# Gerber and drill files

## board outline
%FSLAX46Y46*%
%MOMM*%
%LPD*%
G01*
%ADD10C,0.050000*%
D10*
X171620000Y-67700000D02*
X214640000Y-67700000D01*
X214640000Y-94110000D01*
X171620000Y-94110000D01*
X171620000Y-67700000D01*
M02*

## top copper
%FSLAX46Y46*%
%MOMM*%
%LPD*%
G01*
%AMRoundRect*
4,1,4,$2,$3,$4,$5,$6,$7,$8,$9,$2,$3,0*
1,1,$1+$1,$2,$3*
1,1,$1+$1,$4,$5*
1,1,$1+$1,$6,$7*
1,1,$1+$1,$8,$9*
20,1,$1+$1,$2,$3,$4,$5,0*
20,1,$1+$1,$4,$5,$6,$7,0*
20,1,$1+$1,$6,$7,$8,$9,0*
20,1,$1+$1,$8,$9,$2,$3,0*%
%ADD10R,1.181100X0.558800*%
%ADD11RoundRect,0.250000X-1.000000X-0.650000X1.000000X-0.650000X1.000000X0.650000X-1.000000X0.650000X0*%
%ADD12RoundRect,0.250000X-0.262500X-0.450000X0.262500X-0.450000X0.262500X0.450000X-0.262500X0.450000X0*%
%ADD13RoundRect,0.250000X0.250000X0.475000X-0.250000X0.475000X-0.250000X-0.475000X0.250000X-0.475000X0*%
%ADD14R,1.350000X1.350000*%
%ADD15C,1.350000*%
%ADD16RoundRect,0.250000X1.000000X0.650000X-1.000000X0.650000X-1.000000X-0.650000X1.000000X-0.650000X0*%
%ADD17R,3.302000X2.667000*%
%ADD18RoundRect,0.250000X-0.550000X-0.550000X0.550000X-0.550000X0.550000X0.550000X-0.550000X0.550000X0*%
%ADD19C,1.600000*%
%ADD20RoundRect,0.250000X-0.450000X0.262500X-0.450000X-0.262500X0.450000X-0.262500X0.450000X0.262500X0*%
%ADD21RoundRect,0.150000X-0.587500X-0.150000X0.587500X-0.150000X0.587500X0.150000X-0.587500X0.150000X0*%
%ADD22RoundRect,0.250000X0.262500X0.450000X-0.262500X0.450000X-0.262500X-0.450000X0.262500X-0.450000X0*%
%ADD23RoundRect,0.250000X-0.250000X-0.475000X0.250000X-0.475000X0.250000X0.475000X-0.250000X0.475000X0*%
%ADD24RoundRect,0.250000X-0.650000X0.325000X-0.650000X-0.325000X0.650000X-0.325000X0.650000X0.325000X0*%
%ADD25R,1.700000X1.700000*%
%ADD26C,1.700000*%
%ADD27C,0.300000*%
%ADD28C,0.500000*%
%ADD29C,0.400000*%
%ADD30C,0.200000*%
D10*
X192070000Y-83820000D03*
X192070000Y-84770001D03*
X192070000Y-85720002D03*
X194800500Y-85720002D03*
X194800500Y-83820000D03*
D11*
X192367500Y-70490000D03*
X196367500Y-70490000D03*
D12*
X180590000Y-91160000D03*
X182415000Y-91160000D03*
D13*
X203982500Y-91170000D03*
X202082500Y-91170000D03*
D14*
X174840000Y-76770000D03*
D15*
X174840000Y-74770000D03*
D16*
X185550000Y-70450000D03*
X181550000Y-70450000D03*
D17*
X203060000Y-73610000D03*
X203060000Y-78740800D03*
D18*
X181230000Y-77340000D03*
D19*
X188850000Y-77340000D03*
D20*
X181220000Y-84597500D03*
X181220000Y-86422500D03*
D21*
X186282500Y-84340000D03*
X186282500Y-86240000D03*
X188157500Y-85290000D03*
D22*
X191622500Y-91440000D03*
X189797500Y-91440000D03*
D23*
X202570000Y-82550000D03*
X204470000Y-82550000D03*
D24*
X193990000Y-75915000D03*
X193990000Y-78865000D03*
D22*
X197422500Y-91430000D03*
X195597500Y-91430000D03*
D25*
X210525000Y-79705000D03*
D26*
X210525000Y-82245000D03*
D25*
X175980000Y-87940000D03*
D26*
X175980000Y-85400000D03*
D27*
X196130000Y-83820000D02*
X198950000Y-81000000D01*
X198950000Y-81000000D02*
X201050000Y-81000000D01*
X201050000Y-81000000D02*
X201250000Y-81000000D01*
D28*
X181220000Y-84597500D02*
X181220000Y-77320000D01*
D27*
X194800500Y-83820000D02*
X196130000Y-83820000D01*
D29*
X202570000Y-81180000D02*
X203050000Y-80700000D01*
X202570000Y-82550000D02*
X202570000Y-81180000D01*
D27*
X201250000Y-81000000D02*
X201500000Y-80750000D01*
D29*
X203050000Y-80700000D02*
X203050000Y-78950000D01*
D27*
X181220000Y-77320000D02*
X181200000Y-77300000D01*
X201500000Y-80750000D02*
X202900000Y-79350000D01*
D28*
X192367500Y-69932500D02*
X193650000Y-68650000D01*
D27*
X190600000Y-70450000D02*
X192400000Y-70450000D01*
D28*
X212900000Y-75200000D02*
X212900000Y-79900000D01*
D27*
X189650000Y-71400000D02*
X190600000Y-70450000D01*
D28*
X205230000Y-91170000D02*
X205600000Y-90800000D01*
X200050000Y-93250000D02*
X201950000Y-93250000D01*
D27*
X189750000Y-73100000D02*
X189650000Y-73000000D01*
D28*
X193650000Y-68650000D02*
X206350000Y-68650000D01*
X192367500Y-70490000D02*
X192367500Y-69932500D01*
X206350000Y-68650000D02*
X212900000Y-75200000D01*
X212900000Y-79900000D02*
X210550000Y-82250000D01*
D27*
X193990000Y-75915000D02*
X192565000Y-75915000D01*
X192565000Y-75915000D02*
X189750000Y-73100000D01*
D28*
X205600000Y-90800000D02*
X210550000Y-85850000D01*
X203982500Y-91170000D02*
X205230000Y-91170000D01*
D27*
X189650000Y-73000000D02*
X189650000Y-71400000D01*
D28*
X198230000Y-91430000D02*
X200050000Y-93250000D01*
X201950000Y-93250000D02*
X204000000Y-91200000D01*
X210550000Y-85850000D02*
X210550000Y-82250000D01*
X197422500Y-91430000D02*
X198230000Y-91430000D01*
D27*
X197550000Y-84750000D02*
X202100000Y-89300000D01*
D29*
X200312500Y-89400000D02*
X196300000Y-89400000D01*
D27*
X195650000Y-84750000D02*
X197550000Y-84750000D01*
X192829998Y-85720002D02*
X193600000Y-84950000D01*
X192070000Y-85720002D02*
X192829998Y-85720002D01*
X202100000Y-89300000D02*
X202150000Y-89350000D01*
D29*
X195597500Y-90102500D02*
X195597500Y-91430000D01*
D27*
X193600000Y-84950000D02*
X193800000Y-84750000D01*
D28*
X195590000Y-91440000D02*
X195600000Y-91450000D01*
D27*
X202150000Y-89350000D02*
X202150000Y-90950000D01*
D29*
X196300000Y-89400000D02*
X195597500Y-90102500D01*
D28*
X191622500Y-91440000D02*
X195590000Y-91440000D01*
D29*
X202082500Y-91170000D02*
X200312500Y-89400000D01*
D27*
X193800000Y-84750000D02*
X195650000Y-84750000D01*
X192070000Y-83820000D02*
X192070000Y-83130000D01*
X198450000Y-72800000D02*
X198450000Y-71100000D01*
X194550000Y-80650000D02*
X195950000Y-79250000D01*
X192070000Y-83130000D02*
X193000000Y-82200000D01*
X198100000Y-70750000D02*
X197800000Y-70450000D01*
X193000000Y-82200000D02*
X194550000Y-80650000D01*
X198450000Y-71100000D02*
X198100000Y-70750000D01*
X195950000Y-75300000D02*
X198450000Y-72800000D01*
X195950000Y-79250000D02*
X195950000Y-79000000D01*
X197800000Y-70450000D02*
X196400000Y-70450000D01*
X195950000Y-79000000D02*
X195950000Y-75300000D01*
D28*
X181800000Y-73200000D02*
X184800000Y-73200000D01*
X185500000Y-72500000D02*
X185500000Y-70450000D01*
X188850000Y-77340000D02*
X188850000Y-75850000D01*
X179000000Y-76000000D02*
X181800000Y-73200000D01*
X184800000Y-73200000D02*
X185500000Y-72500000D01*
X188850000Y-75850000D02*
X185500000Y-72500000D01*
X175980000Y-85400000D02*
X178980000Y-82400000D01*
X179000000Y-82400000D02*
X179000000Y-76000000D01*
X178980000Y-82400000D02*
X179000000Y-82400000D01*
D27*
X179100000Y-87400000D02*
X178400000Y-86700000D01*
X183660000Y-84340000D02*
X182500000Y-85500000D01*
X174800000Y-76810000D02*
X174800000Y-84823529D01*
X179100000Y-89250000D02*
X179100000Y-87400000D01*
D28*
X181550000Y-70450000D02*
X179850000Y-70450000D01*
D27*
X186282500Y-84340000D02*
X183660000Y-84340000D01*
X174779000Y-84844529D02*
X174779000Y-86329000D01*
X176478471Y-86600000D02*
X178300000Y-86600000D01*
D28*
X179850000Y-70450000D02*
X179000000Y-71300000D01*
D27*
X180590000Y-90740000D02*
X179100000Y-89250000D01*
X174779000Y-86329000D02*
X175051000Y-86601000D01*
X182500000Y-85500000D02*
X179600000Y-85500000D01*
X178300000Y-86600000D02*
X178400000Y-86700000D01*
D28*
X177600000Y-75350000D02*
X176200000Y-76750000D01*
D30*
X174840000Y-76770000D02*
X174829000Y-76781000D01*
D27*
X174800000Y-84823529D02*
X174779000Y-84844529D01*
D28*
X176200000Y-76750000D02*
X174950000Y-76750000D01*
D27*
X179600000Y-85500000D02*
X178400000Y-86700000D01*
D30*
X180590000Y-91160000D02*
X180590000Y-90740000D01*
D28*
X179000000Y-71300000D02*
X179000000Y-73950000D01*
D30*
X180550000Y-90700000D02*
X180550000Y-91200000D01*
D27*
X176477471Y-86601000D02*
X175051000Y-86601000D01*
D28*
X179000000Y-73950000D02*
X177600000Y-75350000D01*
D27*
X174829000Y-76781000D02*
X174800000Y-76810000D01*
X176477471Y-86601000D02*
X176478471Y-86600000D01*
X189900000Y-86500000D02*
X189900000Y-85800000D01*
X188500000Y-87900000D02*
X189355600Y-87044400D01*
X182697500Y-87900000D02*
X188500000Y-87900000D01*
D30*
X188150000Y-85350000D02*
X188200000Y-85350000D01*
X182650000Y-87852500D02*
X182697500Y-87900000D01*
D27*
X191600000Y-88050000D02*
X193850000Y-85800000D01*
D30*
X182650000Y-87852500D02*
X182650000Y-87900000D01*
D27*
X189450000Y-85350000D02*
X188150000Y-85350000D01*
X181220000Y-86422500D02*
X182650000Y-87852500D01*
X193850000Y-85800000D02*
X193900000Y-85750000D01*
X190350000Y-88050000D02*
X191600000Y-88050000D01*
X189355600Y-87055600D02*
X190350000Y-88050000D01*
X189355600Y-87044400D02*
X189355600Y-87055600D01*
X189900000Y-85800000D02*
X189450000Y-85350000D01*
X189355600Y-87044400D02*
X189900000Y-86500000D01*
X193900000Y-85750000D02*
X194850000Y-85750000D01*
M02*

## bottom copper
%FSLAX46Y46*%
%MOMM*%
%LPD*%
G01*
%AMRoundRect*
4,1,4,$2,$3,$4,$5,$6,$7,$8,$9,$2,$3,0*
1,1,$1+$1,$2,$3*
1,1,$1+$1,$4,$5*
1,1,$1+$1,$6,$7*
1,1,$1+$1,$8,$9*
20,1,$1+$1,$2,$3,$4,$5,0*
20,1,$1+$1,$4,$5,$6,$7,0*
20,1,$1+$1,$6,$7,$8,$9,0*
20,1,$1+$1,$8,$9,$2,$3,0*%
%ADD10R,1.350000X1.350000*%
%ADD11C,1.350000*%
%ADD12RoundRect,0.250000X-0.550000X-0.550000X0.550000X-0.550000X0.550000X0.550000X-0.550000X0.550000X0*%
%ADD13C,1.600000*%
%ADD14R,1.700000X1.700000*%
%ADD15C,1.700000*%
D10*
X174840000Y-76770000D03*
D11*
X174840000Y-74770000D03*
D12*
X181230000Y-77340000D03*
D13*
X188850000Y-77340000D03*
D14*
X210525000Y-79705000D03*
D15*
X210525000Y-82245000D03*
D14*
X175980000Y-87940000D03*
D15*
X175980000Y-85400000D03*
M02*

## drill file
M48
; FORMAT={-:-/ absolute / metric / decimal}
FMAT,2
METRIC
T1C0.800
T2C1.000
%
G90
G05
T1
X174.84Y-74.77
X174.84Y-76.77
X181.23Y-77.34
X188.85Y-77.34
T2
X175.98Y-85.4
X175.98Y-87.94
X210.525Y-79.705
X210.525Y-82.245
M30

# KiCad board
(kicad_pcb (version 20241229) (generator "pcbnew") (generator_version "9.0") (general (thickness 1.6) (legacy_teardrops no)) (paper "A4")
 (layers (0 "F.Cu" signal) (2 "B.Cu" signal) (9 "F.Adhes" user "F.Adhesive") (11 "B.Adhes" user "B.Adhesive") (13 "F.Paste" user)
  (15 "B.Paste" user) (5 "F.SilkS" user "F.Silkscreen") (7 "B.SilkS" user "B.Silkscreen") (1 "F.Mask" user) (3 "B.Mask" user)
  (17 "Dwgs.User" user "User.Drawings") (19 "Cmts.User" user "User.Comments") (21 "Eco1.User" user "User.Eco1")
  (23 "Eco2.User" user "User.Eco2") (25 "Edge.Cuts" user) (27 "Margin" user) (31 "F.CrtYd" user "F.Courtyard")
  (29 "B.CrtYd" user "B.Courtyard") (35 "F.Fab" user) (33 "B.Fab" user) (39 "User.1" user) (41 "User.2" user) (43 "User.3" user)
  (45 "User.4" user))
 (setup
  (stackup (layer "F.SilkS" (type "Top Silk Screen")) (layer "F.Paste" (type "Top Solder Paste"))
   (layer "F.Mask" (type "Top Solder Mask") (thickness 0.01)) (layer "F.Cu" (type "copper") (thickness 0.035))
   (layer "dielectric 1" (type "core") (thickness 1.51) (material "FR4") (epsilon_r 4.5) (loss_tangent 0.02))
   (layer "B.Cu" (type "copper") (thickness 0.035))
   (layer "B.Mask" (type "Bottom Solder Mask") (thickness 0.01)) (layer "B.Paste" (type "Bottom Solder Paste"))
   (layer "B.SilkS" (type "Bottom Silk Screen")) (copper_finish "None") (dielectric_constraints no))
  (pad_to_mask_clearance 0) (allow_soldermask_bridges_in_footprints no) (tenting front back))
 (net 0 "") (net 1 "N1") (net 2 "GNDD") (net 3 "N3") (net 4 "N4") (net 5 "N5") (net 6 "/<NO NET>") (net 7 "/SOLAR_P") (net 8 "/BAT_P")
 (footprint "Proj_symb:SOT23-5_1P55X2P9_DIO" (layer "F.Cu") (at 193.43525 84.770001)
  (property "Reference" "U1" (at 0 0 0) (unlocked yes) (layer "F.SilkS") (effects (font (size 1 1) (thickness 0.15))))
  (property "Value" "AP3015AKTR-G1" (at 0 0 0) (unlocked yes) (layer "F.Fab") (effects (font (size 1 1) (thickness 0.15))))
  (pad "1" smd rect (at -1.36525 -0.950001) (size 1.1811 0.5588) (layers "F.Cu" "F.Mask" "F.Paste") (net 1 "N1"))
  (pad "2" smd rect (at -1.36525 0) (size 1.1811 0.5588) (layers "F.Cu" "F.Mask" "F.Paste") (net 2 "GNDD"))
  (pad "3" smd rect (at -1.36525 0.950001) (size 1.1811 0.5588) (layers "F.Cu" "F.Mask" "F.Paste") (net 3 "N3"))
  (pad "4" smd rect (at 1.36525 0.950001) (size 1.1811 0.5588) (layers "F.Cu" "F.Mask" "F.Paste") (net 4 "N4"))
  (pad "5" smd rect (at 1.36525 -0.950001) (size 1.1811 0.5588) (layers "F.Cu" "F.Mask" "F.Paste") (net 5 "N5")))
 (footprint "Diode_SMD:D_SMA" (layer "F.Cu") (at 194.3675 70.49)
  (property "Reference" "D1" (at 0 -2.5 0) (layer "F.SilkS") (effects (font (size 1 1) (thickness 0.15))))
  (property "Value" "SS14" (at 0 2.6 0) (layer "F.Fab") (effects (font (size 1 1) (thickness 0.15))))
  (pad "1" smd roundrect (at -2 0) (size 2.5 1.8) (layers "F.Cu" "F.Mask" "F.Paste") (roundrect_rratio 0.1388888889) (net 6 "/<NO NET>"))
  (pad "2" smd roundrect (at 2 0) (size 2.5 1.8) (layers "F.Cu" "F.Mask" "F.Paste") (roundrect_rratio 0.1388888889) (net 1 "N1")))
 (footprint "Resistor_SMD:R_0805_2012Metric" (layer "F.Cu") (at 181.5025 91.16)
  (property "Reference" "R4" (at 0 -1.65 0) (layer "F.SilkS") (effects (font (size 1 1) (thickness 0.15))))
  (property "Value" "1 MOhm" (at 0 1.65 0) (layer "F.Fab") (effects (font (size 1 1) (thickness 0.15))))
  (pad "1" smd roundrect (at -0.9125 0) (size 1.025 1.4) (layers "F.Cu" "F.Mask" "F.Paste") (roundrect_rratio 0.243902) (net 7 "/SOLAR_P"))
  (pad "2" smd roundrect (at 0.9125 0) (size 1.025 1.4) (layers "F.Cu" "F.Mask" "F.Paste") (roundrect_rratio 0.243902) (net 2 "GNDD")))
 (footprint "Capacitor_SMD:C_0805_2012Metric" (layer "F.Cu") (at 203.0325 91.17 180)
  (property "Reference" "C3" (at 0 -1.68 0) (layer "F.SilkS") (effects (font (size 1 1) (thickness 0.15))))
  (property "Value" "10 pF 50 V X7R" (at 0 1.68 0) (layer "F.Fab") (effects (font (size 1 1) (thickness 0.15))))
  (pad "1" smd roundrect (at -0.95 0 180) (size 1 1.45) (layers "F.Cu" "F.Mask" "F.Paste") (roundrect_rratio 0.25) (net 6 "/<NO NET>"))
  (pad "2" smd roundrect (at 0.95 0 180) (size 1 1.45) (layers "F.Cu" "F.Mask" "F.Paste") (roundrect_rratio 0.25) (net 3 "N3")))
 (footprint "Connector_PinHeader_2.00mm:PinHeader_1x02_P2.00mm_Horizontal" (layer "F.Cu") (at 174.84 76.77 180)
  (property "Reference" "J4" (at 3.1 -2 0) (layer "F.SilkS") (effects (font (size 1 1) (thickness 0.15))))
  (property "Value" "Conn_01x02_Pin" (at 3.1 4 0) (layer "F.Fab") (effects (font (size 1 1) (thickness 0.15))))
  (pad "1" thru_hole rect (at 0 0 180) (size 1.35 1.35) (drill 0.8) (layers "*.Cu" "*.Mask") (remove_unused_layers no) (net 7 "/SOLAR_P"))
  (pad "2" thru_hole circle (at 0 2 180) (size 1.35 1.35) (drill 0.8) (layers "*.Cu" "*.Mask") (remove_unused_layers no) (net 2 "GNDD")))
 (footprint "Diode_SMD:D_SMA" (layer "F.Cu") (at 183.55 70.45 180)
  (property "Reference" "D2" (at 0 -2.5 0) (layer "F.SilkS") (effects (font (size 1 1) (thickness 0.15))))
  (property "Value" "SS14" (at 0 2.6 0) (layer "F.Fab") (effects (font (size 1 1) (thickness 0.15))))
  (pad "1" smd roundrect (at -2 0 180) (size 2.5 1.8) (layers "F.Cu" "F.Mask" "F.Paste") (roundrect_rratio 0.1388888889) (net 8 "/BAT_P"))
  (pad "2" smd roundrect (at 2 0 180) (size 2.5 1.8) (layers "F.Cu" "F.Mask" "F.Paste") (roundrect_rratio 0.1388888889) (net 7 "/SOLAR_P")))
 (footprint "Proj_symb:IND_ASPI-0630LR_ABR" (layer "F.Cu") (at 203.06 76.1754 -90)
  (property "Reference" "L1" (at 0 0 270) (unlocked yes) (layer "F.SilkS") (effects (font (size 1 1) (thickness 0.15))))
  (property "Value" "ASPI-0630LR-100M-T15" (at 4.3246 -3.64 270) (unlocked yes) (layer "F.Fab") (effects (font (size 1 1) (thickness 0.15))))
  (pad "1" smd rect (at -2.5654 0) (size 3.302 2.667) (layers "F.Cu" "F.Mask" "F.Paste") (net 1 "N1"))
  (pad "2" smd rect (at 2.5654 0) (size 3.302 2.667) (layers "F.Cu" "F.Mask" "F.Paste") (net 5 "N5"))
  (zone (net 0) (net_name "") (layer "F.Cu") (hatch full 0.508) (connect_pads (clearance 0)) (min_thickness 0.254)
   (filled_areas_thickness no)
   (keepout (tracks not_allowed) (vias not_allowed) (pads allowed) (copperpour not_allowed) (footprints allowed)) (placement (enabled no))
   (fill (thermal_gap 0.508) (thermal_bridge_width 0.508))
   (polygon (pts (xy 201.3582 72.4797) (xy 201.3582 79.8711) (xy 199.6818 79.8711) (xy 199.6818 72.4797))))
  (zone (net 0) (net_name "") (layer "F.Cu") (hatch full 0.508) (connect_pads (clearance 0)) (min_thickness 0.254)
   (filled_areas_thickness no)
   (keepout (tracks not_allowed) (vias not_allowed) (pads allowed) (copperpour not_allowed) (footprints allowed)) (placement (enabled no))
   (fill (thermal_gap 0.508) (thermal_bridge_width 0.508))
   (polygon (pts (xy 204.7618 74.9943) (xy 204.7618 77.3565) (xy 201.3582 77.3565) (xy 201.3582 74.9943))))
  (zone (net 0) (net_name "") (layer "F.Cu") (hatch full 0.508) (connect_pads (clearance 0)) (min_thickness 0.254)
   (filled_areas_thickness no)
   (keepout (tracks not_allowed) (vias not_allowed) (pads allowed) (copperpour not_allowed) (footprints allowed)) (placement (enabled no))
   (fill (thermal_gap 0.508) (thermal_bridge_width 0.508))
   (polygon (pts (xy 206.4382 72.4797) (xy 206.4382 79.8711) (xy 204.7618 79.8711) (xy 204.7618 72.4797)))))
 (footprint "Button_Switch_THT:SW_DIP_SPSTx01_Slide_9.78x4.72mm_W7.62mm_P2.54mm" (layer "F.Cu") (at 181.23 77.34)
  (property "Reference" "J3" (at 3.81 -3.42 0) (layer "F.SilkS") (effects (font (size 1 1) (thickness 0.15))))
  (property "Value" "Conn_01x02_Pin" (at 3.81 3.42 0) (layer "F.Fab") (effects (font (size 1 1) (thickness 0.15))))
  (pad "1" thru_hole roundrect (at 0 0) (size 1.6 1.6) (drill 0.8) (layers "*.Cu" "*.Mask") (remove_unused_layers no)
   (roundrect_rratio 0.15625) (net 5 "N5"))
  (pad "2" thru_hole circle (at 7.62 0) (size 1.6 1.6) (drill 0.8) (layers "*.Cu" "*.Mask") (remove_unused_layers no) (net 8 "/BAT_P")))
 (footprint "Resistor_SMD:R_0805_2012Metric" (layer "F.Cu") (at 181.22 85.51 -90)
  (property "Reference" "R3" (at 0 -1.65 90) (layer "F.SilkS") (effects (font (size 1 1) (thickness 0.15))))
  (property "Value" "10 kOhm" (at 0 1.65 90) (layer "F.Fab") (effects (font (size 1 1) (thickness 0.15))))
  (pad "1" smd roundrect (at -0.9125 0 270) (size 1.025 1.4) (layers "F.Cu" "F.Mask" "F.Paste") (roundrect_rratio 0.243902) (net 5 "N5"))
  (pad "2" smd roundrect (at 0.9125 0 270) (size 1.025 1.4) (layers "F.Cu" "F.Mask" "F.Paste") (roundrect_rratio 0.243902) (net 4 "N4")))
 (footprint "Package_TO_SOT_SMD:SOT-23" (layer "F.Cu") (at 187.22 85.29)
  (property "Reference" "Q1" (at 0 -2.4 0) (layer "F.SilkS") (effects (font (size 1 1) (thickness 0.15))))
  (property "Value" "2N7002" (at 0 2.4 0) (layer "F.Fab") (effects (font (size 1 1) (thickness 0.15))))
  (pad "1" smd roundrect (at -0.9375 -0.95) (size 1.475 0.6) (layers "F.Cu" "F.Mask" "F.Paste") (roundrect_rratio 0.25) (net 7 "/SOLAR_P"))
  (pad "2" smd roundrect (at -0.9375 0.95) (size 1.475 0.6) (layers "F.Cu" "F.Mask" "F.Paste") (roundrect_rratio 0.25) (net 2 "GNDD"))
  (pad "3" smd roundrect (at 0.9375 0) (size 1.475 0.6) (layers "F.Cu" "F.Mask" "F.Paste") (roundrect_rratio 0.25) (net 4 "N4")))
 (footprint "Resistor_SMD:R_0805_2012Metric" (layer "F.Cu") (at 190.71 91.44 180)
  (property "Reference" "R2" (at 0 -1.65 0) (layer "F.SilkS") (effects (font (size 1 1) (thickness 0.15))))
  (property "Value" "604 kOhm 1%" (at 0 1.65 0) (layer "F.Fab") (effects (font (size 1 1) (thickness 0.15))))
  (pad "1" smd roundrect (at -0.9125 0 180) (size 1.025 1.4) (layers "F.Cu" "F.Mask" "F.Paste") (roundrect_rratio 0.243902) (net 3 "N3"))
  (pad "2" smd roundrect (at 0.9125 0 180) (size 1.025 1.4) (layers "F.Cu" "F.Mask" "F.Paste") (roundrect_rratio 0.243902) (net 2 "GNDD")))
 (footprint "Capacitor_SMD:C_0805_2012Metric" (layer "F.Cu") (at 203.52 82.55)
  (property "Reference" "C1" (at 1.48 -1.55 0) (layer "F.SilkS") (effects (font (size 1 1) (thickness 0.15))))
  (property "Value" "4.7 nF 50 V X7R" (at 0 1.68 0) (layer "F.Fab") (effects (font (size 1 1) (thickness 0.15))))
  (pad "1" smd roundrect (at -0.95 0) (size 1 1.45) (layers "F.Cu" "F.Mask" "F.Paste") (roundrect_rratio 0.25) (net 5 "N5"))
  (pad "2" smd roundrect (at 0.95 0) (size 1 1.45) (layers "F.Cu" "F.Mask" "F.Paste") (roundrect_rratio 0.25) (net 2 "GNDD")))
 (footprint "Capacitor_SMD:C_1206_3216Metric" (layer "F.Cu") (at 193.99 77.39 -90)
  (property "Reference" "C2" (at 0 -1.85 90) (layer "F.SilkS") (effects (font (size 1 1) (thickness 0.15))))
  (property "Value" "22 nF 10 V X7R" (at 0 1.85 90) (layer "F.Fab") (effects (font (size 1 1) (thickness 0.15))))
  (pad "1" smd roundrect (at -1.475 0 270) (size 1.15 1.8) (layers "F.Cu" "F.Mask" "F.Paste") (roundrect_rratio 0.217391)
   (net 6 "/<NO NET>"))
  (pad "2" smd roundrect (at 1.475 0 270) (size 1.15 1.8) (layers "F.Cu" "F.Mask" "F.Paste") (roundrect_rratio 0.217391) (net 2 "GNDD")))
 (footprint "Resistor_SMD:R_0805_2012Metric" (layer "F.Cu") (at 196.51 91.43 180)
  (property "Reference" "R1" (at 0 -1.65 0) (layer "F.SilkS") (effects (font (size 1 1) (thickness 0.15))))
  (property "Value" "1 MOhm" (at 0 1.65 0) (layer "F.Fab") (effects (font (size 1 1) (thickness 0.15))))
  (pad "1" smd roundrect (at -0.9125 0 180) (size 1.025 1.4) (layers "F.Cu" "F.Mask" "F.Paste") (roundrect_rratio 0.243902)
   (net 6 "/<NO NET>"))
  (pad "2" smd roundrect (at 0.9125 0 180) (size 1.025 1.4) (layers "F.Cu" "F.Mask" "F.Paste") (roundrect_rratio 0.243902) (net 3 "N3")))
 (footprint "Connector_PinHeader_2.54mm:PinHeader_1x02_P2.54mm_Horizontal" (layer "F.Cu") (at 210.525 79.705)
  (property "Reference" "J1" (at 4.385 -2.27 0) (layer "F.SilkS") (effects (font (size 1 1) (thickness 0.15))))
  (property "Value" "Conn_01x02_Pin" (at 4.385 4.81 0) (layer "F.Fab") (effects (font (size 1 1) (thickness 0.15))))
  (pad "1" thru_hole rect (at 0 0) (size 1.7 1.7) (drill 1) (layers "*.Cu" "*.Mask") (remove_unused_layers no) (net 2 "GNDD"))
  (pad "2" thru_hole circle (at 0 2.54) (size 1.7 1.7) (drill 1) (layers "*.Cu" "*.Mask") (remove_unused_layers no) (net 6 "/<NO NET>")))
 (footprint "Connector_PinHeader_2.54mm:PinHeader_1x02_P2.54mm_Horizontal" (layer "F.Cu") (at 175.98 87.94 180)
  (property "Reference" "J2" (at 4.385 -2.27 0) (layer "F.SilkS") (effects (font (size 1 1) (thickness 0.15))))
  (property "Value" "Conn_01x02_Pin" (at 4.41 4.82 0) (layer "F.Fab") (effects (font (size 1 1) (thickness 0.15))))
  (pad "1" thru_hole rect (at 0 0 180) (size 1.7 1.7) (drill 1) (layers "*.Cu" "*.Mask") (remove_unused_layers no) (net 2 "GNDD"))
  (pad "2" thru_hole circle (at 0 2.54 180) (size 1.7 1.7) (drill 1) (layers "*.Cu" "*.Mask") (remove_unused_layers no) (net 8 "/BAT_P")))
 (gr_rect (start 171.62 67.7) (end 214.64 94.11) (stroke (width 0.05) (type default)) (fill no) (layer "Edge.Cuts"))
 (segment (start 196.13 83.82) (end 198.95 81) (width 0.3) (layer "F.Cu") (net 5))
 (segment (start 198.95 81) (end 201.05 81) (width 0.3) (layer "F.Cu") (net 5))
 (segment (start 201.05 81) (end 201.25 81) (width 0.3) (layer "F.Cu") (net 5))
 (segment (start 181.22 84.5975) (end 181.22 77.32) (width 0.5) (layer "F.Cu") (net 5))
 (segment (start 194.8005 83.82) (end 196.13 83.82) (width 0.3) (layer "F.Cu") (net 5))
 (segment (start 202.57 81.18) (end 203.05 80.7) (width 0.4) (layer "F.Cu") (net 5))
 (segment (start 202.57 82.55) (end 202.57 81.18) (width 0.4) (layer "F.Cu") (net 5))
 (segment (start 201.25 81) (end 201.5 80.75) (width 0.3) (layer "F.Cu") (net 5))
 (segment (start 203.05 80.7) (end 203.05 78.95) (width 0.4) (layer "F.Cu") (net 5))
 (segment (start 181.22 77.32) (end 181.2 77.3) (width 0.3) (layer "F.Cu") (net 5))
 (segment (start 201.5 80.75) (end 202.9 79.35) (width 0.3) (layer "F.Cu") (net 5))
 (segment (start 192.3675 69.9325) (end 193.65 68.65) (width 0.5) (layer "F.Cu") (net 6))
 (segment (start 190.6 70.45) (end 192.4 70.45) (width 0.3) (layer "F.Cu") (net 6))
 (segment (start 212.9 75.2) (end 212.9 79.9) (width 0.5) (layer "F.Cu") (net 6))
 (segment (start 189.65 71.4) (end 190.6 70.45) (width 0.3) (layer "F.Cu") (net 6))
 (segment (start 205.23 91.17) (end 205.6 90.8) (width 0.5) (layer "F.Cu") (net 6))
 (segment (start 200.05 93.25) (end 201.95 93.25) (width 0.5) (layer "F.Cu") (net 6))
 (segment (start 189.75 73.1) (end 189.65 73) (width 0.3) (layer "F.Cu") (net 6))
 (segment (start 193.65 68.65) (end 206.35 68.65) (width 0.5) (layer "F.Cu") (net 6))
 (segment (start 192.3675 70.49) (end 192.3675 69.9325) (width 0.5) (layer "F.Cu") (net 6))
 (segment (start 206.35 68.65) (end 212.9 75.2) (width 0.5) (layer "F.Cu") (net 6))
 (segment (start 212.9 79.9) (end 210.55 82.25) (width 0.5) (layer "F.Cu") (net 6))
 (segment (start 193.99 75.915) (end 192.565 75.915) (width 0.3) (layer "F.Cu") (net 6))
 (segment (start 192.565 75.915) (end 189.75 73.1) (width 0.3) (layer "F.Cu") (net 6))
 (segment (start 205.6 90.8) (end 210.55 85.85) (width 0.5) (layer "F.Cu") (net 6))
 (segment (start 203.9825 91.17) (end 205.23 91.17) (width 0.5) (layer "F.Cu") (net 6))
 (segment (start 189.65 73) (end 189.65 71.4) (width 0.3) (layer "F.Cu") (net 6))
 (segment (start 198.23 91.43) (end 200.05 93.25) (width 0.5) (layer "F.Cu") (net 6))
 (segment (start 201.95 93.25) (end 204 91.2) (width 0.5) (layer "F.Cu") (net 6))
 (segment (start 210.55 85.85) (end 210.55 82.25) (width 0.5) (layer "F.Cu") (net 6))
 (segment (start 197.4225 91.43) (end 198.23 91.43) (width 0.5) (layer "F.Cu") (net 6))
 (segment (start 197.55 84.75) (end 202.1 89.3) (width 0.3) (layer "F.Cu") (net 3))
 (segment (start 200.3125 89.4) (end 196.3 89.4) (width 0.4) (layer "F.Cu") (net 3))
 (segment (start 195.65 84.75) (end 197.55 84.75) (width 0.3) (layer "F.Cu") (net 3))
 (segment (start 192.829998 85.720002) (end 193.6 84.95) (width 0.3) (layer "F.Cu") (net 3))
 (segment (start 192.07 85.720002) (end 192.829998 85.720002) (width 0.3) (layer "F.Cu") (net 3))
 (segment (start 202.1 89.3) (end 202.15 89.35) (width 0.3) (layer "F.Cu") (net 3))
 (segment (start 195.5975 90.1025) (end 195.5975 91.43) (width 0.4) (layer "F.Cu") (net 3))
 (segment (start 193.6 84.95) (end 193.8 84.75) (width 0.3) (layer "F.Cu") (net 3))
 (segment (start 195.59 91.44) (end 195.6 91.45) (width 0.5) (layer "F.Cu") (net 3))
 (segment (start 202.15 89.35) (end 202.15 90.95) (width 0.3) (layer "F.Cu") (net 3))
 (segment (start 196.3 89.4) (end 195.5975 90.1025) (width 0.4) (layer "F.Cu") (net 3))
 (segment (start 191.6225 91.44) (end 195.59 91.44) (width 0.5) (layer "F.Cu") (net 3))
 (segment (start 202.0825 91.17) (end 200.3125 89.4) (width 0.4) (layer "F.Cu") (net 3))
 (segment (start 193.8 84.75) (end 195.65 84.75) (width 0.3) (layer "F.Cu") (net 3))
 (segment (start 192.07 83.82) (end 192.07 83.13) (width 0.3) (layer "F.Cu") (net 1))
 (segment (start 198.45 72.8) (end 198.45 71.1) (width 0.3) (layer "F.Cu") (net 1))
 (segment (start 194.55 80.65) (end 195.95 79.25) (width 0.3) (layer "F.Cu") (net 1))
 (segment (start 192.07 83.13) (end 193 82.2) (width 0.3) (layer "F.Cu") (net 1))
 (segment (start 198.1 70.75) (end 197.8 70.45) (width 0.3) (layer "F.Cu") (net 1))
 (segment (start 193 82.2) (end 194.55 80.65) (width 0.3) (layer "F.Cu") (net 1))
 (segment (start 198.45 71.1) (end 198.1 70.75) (width 0.3) (layer "F.Cu") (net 1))
 (segment (start 195.95 75.3) (end 198.45 72.8) (width 0.3) (layer "F.Cu") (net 1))
 (segment (start 195.95 79.25) (end 195.95 79) (width 0.3) (layer "F.Cu") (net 1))
 (segment (start 197.8 70.45) (end 196.4 70.45) (width 0.3) (layer "F.Cu") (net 1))
 (segment (start 195.95 79) (end 195.95 75.3) (width 0.3) (layer "F.Cu") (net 1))
 (segment (start 181.8 73.2) (end 184.8 73.2) (width 0.5) (layer "F.Cu") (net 8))
 (segment (start 185.5 72.5) (end 185.5 70.45) (width 0.5) (layer "F.Cu") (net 8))
 (segment (start 188.85 77.34) (end 188.85 75.85) (width 0.5) (layer "F.Cu") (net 8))
 (segment (start 179 76) (end 181.8 73.2) (width 0.5) (layer "F.Cu") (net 8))
 (segment (start 184.8 73.2) (end 185.5 72.5) (width 0.5) (layer "F.Cu") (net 8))
 (segment (start 188.85 75.85) (end 185.5 72.5) (width 0.5) (layer "F.Cu") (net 8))
 (segment (start 175.98 85.4) (end 178.98 82.4) (width 0.5) (layer "F.Cu") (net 8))
 (segment (start 179 82.4) (end 179 76) (width 0.5) (layer "F.Cu") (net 8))
 (segment (start 178.98 82.4) (end 179 82.4) (width 0.5) (layer "F.Cu") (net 8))
 (segment (start 179.1 87.4) (end 178.4 86.7) (width 0.3) (layer "F.Cu") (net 7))
 (segment (start 183.66 84.34) (end 182.5 85.5) (width 0.3) (layer "F.Cu") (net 7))
 (segment (start 174.8 76.81) (end 174.8 84.823529) (width 0.3) (layer "F.Cu") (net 7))
 (segment (start 179.1 89.25) (end 179.1 87.4) (width 0.3) (layer "F.Cu") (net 7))
 (segment (start 181.55 70.45) (end 179.85 70.45) (width 0.5) (layer "F.Cu") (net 7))
 (segment (start 186.2825 84.34) (end 183.66 84.34) (width 0.3) (layer "F.Cu") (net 7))
 (segment (start 174.779 84.844529) (end 174.779 86.329) (width 0.3) (layer "F.Cu") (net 7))
 (segment (start 176.478471 86.6) (end 178.3 86.6) (width 0.3) (layer "F.Cu") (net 7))
 (segment (start 179.85 70.45) (end 179 71.3) (width 0.5) (layer "F.Cu") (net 7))
 (segment (start 180.59 90.74) (end 179.1 89.25) (width 0.3) (layer "F.Cu") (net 7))
 (segment (start 174.779 86.329) (end 175.051 86.601) (width 0.3) (layer "F.Cu") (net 7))
 (segment (start 182.5 85.5) (end 179.6 85.5) (width 0.3) (layer "F.Cu") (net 7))
 (segment (start 178.3 86.6) (end 178.4 86.7) (width 0.3) (layer "F.Cu") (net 7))
 (segment (start 177.6 75.35) (end 176.2 76.75) (width 0.5) (layer "F.Cu") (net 7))
 (segment (start 174.84 76.77) (end 174.829 76.781) (width 0.2) (layer "F.Cu") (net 7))
 (segment (start 174.8 84.823529) (end 174.779 84.844529) (width 0.3) (layer "F.Cu") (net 7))
 (segment (start 176.2 76.75) (end 174.95 76.75) (width 0.5) (layer "F.Cu") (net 7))
 (segment (start 179.6 85.5) (end 178.4 86.7) (width 0.3) (layer "F.Cu") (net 7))
 (segment (start 180.59 91.16) (end 180.59 90.74) (width 0.2) (layer "F.Cu") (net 7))
 (segment (start 179 71.3) (end 179 73.95) (width 0.5) (layer "F.Cu") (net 7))
 (segment (start 180.55 90.7) (end 180.55 91.2) (width 0.2) (layer "F.Cu") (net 7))
 (segment (start 176.477471 86.601) (end 175.051 86.601) (width 0.3) (layer "F.Cu") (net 7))
 (segment (start 179 73.95) (end 177.6 75.35) (width 0.5) (layer "F.Cu") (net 7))
 (segment (start 174.829 76.781) (end 174.8 76.81) (width 0.3) (layer "F.Cu") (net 7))
 (segment (start 176.477471 86.601) (end 176.478471 86.6) (width 0.3) (layer "F.Cu") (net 7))
 (segment (start 189.9 86.5) (end 189.9 85.8) (width 0.3) (layer "F.Cu") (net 4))
 (segment (start 188.5 87.9) (end 189.3556 87.0444) (width 0.3) (layer "F.Cu") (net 4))
 (segment (start 182.6975 87.9) (end 188.5 87.9) (width 0.3) (layer "F.Cu") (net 4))
 (segment (start 188.15 85.35) (end 188.2 85.35) (width 0.2) (layer "F.Cu") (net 4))
 (segment (start 182.65 87.8525) (end 182.6975 87.9) (width 0.2) (layer "F.Cu") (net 4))
 (segment (start 191.6 88.05) (end 193.85 85.8) (width 0.3) (layer "F.Cu") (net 4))
 (segment (start 182.65 87.8525) (end 182.65 87.9) (width 0.2) (layer "F.Cu") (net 4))
 (segment (start 189.45 85.35) (end 188.15 85.35) (width 0.3) (layer "F.Cu") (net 4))
 (segment (start 181.22 86.4225) (end 182.65 87.8525) (width 0.3) (layer "F.Cu") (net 4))
 (segment (start 193.85 85.8) (end 193.9 85.75) (width 0.3) (layer "F.Cu") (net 4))
 (segment (start 190.35 88.05) (end 191.6 88.05) (width 0.3) (layer "F.Cu") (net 4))
 (segment (start 189.3556 87.0556) (end 190.35 88.05) (width 0.3) (layer "F.Cu") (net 4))
 (segment (start 189.3556 87.0444) (end 189.3556 87.0556) (width 0.3) (layer "F.Cu") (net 4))
 (segment (start 189.9 85.8) (end 189.45 85.35) (width 0.3) (layer "F.Cu") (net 4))
 (segment (start 189.3556 87.0444) (end 189.9 86.5) (width 0.3) (layer "F.Cu") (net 4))
 (segment (start 193.9 85.75) (end 194.85 85.75) (width 0.3) (layer "F.Cu") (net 4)))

